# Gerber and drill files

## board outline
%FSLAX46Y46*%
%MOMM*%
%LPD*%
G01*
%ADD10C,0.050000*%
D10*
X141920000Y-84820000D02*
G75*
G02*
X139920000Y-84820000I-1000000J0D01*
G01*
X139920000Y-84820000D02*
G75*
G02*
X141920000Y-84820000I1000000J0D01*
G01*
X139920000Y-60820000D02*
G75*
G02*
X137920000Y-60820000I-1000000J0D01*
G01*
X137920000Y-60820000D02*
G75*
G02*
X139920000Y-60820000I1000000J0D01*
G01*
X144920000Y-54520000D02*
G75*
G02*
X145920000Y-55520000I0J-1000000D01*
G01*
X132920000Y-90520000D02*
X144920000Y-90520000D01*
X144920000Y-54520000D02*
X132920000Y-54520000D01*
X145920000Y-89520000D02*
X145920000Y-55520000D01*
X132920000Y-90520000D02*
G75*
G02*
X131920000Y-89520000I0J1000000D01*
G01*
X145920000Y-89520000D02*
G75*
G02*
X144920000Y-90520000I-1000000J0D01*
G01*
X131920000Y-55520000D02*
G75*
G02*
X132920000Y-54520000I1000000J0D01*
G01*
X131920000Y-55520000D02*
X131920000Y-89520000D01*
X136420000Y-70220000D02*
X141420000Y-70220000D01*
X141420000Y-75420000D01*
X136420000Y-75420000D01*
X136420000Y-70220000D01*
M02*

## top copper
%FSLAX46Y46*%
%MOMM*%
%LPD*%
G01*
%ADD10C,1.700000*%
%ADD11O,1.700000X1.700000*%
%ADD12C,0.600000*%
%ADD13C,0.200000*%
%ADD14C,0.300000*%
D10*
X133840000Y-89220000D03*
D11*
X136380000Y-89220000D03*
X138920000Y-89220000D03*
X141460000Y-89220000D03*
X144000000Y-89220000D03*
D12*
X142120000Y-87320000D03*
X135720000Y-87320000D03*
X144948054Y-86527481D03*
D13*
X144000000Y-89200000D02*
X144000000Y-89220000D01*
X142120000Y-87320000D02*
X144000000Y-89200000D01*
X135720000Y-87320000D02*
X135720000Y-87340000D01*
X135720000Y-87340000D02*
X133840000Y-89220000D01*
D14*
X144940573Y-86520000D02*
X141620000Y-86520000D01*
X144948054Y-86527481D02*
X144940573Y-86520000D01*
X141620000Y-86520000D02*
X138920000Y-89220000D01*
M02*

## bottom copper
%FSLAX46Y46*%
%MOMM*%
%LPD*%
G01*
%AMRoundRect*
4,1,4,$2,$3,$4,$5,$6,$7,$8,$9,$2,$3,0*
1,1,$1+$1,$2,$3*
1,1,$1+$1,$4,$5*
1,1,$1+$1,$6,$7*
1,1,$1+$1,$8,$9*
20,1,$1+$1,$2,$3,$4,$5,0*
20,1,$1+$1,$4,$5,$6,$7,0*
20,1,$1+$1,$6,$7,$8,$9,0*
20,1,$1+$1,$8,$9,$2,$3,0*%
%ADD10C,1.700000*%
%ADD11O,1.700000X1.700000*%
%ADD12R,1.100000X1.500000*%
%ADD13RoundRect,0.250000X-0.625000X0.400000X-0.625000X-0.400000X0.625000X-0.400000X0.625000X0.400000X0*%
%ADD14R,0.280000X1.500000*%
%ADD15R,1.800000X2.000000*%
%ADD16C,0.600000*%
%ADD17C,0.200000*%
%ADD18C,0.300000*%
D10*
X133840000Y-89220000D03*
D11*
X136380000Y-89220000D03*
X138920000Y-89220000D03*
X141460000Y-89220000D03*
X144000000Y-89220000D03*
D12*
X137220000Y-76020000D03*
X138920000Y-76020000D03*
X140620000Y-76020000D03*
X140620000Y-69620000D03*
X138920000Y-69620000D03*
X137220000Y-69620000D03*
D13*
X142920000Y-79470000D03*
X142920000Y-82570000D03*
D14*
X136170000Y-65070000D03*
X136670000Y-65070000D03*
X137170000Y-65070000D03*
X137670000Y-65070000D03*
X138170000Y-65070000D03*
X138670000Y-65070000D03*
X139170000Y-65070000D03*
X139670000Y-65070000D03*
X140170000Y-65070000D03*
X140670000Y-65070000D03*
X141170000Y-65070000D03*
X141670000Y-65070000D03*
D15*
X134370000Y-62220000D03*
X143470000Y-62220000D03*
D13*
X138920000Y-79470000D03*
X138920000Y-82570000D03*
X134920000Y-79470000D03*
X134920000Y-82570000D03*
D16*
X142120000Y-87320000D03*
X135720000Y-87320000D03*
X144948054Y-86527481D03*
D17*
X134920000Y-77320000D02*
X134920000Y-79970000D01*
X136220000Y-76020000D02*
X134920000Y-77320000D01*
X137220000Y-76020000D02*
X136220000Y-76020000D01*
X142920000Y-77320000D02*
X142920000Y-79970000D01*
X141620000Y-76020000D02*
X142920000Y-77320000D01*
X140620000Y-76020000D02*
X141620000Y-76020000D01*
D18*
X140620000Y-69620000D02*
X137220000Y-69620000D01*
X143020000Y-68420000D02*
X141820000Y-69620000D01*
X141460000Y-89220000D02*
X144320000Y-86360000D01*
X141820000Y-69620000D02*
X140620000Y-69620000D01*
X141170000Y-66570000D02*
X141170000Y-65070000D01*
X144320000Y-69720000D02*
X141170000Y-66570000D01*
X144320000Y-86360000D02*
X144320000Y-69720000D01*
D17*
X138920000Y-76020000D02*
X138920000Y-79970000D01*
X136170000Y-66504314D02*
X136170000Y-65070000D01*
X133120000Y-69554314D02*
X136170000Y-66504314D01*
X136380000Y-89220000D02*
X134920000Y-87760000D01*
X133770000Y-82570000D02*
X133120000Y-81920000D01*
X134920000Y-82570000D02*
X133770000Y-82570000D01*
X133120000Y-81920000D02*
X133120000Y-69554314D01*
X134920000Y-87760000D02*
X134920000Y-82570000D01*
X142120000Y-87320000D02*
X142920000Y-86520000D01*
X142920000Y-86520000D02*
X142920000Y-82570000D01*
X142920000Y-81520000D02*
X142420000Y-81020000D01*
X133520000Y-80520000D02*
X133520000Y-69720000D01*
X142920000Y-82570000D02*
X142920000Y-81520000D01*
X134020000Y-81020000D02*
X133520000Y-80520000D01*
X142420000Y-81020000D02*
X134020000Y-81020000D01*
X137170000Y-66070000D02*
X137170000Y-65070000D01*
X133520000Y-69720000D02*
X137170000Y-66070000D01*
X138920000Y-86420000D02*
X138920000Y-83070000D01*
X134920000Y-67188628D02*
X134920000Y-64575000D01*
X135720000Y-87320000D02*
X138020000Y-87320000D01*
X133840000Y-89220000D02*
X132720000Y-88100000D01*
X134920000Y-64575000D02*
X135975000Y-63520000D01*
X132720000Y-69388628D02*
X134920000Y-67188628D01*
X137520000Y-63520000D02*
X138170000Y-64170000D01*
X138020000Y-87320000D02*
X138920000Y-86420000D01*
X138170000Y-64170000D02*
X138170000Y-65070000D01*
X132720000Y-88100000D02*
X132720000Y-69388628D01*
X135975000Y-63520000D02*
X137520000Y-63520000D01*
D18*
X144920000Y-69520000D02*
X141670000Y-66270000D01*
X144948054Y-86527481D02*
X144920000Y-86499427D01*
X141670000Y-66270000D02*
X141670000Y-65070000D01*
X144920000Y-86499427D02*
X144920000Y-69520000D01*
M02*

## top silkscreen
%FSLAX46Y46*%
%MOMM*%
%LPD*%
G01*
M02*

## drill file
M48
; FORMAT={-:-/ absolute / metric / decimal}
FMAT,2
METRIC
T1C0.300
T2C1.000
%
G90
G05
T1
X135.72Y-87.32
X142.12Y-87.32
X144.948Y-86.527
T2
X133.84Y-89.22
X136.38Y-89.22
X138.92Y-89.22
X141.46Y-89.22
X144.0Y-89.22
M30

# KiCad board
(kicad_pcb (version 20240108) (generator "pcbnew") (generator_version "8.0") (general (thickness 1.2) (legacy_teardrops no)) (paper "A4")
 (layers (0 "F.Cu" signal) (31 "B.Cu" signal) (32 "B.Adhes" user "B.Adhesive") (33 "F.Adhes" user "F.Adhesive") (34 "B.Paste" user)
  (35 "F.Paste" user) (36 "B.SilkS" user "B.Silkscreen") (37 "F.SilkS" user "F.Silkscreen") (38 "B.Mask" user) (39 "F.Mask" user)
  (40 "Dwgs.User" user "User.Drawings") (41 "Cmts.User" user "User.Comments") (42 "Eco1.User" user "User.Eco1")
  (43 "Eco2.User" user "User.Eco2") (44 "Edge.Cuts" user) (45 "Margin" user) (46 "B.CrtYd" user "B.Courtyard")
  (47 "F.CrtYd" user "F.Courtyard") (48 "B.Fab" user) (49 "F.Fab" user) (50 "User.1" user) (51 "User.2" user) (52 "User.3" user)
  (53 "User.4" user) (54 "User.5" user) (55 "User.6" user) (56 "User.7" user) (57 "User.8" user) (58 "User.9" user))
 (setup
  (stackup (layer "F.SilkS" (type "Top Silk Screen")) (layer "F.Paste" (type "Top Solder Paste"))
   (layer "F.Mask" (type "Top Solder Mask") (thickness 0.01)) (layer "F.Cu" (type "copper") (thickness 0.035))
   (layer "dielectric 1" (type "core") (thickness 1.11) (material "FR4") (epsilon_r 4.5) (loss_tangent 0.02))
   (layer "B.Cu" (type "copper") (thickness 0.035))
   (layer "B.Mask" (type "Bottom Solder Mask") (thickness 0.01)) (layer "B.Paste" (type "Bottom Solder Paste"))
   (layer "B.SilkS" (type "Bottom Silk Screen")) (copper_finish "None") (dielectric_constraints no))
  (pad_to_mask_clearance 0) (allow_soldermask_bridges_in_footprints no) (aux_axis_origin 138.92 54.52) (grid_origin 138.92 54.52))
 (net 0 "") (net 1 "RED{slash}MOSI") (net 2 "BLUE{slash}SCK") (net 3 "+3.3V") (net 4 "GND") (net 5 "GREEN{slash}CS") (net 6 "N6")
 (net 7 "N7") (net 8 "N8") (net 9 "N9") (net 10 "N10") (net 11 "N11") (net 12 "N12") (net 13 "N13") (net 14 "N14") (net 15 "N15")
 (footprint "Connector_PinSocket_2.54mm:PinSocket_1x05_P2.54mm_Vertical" (layer "F.Cu") (at 133.84 89.22 90)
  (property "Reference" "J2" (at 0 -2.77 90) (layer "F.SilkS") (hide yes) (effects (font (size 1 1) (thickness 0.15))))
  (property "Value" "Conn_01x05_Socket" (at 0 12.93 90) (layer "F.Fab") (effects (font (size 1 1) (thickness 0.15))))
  (pad "1" thru_hole circle (at 0 0 90) (size 1.7 1.7) (drill 1) (layers "*.Cu" "*.Mask") (remove_unused_layers no) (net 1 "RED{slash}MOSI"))
  (pad "2" thru_hole oval (at 0 2.54 90) (size 1.7 1.7) (drill 1) (layers "*.Cu" "*.Mask") (remove_unused_layers no)
   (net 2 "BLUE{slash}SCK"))
  (pad "3" thru_hole oval (at 0 5.08 90) (size 1.7 1.7) (drill 1) (layers "*.Cu" "*.Mask") (remove_unused_layers no) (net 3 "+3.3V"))
  (pad "4" thru_hole oval (at 0 7.62 90) (size 1.7 1.7) (drill 1) (layers "*.Cu" "*.Mask") (remove_unused_layers no) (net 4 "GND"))
  (pad "5" thru_hole oval (at 0 10.16 90) (size 1.7 1.7) (drill 1) (layers "*.Cu" "*.Mask") (remove_unused_layers no)
   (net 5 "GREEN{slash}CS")))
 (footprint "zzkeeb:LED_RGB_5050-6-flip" (layer "F.Cu") (at 138.92 72.82 90)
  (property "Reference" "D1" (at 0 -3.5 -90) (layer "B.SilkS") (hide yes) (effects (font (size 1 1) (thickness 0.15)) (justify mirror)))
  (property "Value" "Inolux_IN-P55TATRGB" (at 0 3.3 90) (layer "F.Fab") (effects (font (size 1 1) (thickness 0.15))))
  (fp_rect (start -2.6 -2.5) (end 2.6 2.5) (stroke (width 0.05) (type default)) (fill none) (layer "Edge.Cuts"))
  (pad "1" smd rect (at -3.2 -1.7) (size 1.1 1.5) (layers "B.Cu" "B.Paste" "B.Mask") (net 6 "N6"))
  (pad "2" smd rect (at -3.2 0) (size 1.1 1.5) (layers "B.Cu" "B.Paste" "B.Mask") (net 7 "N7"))
  (pad "3" smd rect (at -3.2 1.7) (size 1.1 1.5) (layers "B.Cu" "B.Paste" "B.Mask") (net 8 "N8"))
  (pad "4" smd rect (at 3.2 1.7) (size 1.1 1.5) (layers "B.Cu" "B.Paste" "B.Mask") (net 4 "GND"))
  (pad "5" smd rect (at 3.2 0) (size 1.1 1.5) (layers "B.Cu" "B.Paste" "B.Mask") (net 4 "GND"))
  (pad "6" smd rect (at 3.2 -1.7) (size 1.1 1.5) (layers "B.Cu" "B.Paste" "B.Mask") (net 4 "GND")))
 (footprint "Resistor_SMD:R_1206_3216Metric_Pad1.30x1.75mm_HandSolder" (layer "B.Cu") (at 142.92 81.02 -90)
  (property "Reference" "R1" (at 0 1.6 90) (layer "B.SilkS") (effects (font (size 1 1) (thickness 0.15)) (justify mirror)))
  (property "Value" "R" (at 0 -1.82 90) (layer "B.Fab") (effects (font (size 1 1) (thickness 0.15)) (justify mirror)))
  (pad "1" smd roundrect (at -1.55 0 270) (size 1.3 1.75) (layers "B.Cu" "B.Paste" "B.Mask") (roundrect_rratio 0.192308) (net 8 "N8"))
  (pad "2" smd roundrect (at 1.55 0 270) (size 1.3 1.75) (layers "B.Cu" "B.Paste" "B.Mask") (roundrect_rratio 0.192308)
   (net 5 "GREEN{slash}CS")))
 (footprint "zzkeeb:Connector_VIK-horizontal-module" (layer "B.Cu") (at 138.92 63.52)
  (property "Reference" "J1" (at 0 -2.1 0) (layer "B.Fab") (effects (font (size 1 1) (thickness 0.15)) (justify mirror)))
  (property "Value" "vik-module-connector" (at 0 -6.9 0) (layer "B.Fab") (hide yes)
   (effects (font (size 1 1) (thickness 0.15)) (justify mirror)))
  (pad "1" smd rect (at -2.75 1.55) (size 0.28 1.5) (layers "B.Cu" "B.Paste" "B.Mask") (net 2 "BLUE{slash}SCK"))
  (pad "2" smd rect (at -2.25 1.55) (size 0.28 1.5) (layers "B.Cu" "B.Paste" "B.Mask") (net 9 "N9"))
  (pad "3" smd rect (at -1.75 1.55) (size 0.28 1.5) (layers "B.Cu" "B.Paste" "B.Mask") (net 5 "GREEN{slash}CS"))
  (pad "4" smd rect (at -1.25 1.55) (size 0.28 1.5) (layers "B.Cu" "B.Paste" "B.Mask") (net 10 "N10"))
  (pad "5" smd rect (at -0.75 1.55) (size 0.28 1.5) (layers "B.Cu" "B.Paste" "B.Mask") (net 1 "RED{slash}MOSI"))
  (pad "6" smd rect (at -0.25 1.55) (size 0.28 1.5) (layers "B.Cu" "B.Paste" "B.Mask") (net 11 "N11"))
  (pad "7" smd rect (at 0.25 1.55) (size 0.28 1.5) (layers "B.Cu" "B.Paste" "B.Mask") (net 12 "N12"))
  (pad "8" smd rect (at 0.75 1.55) (size 0.28 1.5) (layers "B.Cu" "B.Paste" "B.Mask") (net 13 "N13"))
  (pad "9" smd rect (at 1.25 1.55) (size 0.28 1.5) (layers "B.Cu" "B.Paste" "B.Mask") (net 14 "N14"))
  (pad "10" smd rect (at 1.75 1.55) (size 0.28 1.5) (layers "B.Cu" "B.Paste" "B.Mask") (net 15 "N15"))
  (pad "11" smd rect (at 2.25 1.55) (size 0.28 1.5) (layers "B.Cu" "B.Paste" "B.Mask") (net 4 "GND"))
  (pad "12" smd rect (at 2.75 1.55) (size 0.28 1.5) (layers "B.Cu" "B.Paste" "B.Mask") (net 3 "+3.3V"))
  (pad "MP" smd rect (at -4.55 -1.3) (size 1.8 2) (layers "B.Cu" "B.Paste" "B.Mask"))
  (pad "MP" smd rect (at 4.55 -1.3) (size 1.8 2) (layers "B.Cu" "B.Paste" "B.Mask")))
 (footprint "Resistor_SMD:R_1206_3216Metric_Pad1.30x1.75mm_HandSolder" (layer "B.Cu") (at 138.92 81.02 -90)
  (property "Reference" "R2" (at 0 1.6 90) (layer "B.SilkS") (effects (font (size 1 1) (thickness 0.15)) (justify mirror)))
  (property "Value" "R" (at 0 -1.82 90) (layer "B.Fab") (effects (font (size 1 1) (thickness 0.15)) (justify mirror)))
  (pad "1" smd roundrect (at -1.55 0 270) (size 1.3 1.75) (layers "B.Cu" "B.Paste" "B.Mask") (roundrect_rratio 0.192308) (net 7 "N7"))
  (pad "2" smd roundrect (at 1.55 0 270) (size 1.3 1.75) (layers "B.Cu" "B.Paste" "B.Mask") (roundrect_rratio 0.192308)
   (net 1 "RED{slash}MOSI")))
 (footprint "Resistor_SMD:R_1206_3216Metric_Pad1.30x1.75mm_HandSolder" (layer "B.Cu") (at 134.92 81.02 -90)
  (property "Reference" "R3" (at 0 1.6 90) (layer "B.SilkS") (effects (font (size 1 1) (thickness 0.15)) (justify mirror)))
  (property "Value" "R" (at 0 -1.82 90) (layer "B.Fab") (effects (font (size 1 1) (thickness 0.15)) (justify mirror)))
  (pad "1" smd roundrect (at -1.55 0 270) (size 1.3 1.75) (layers "B.Cu" "B.Paste" "B.Mask") (roundrect_rratio 0.192308) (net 6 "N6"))
  (pad "2" smd roundrect (at 1.55 0 270) (size 1.3 1.75) (layers "B.Cu" "B.Paste" "B.Mask") (roundrect_rratio 0.192308)
   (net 2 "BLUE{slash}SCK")))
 (gr_circle (center 140.92 84.82) (end 141.92 84.82) (stroke (width 0.05) (type default)) (fill none) (layer "Edge.Cuts"))
 (gr_circle (center 138.92 60.82) (end 139.92 60.82) (stroke (width 0.05) (type default)) (fill none) (layer "Edge.Cuts"))
 (gr_arc (start 144.92 54.52) (mid 145.627107 54.812893) (end 145.92 55.52) (stroke (width 0.05) (type default)) (layer "Edge.Cuts"))
 (gr_line (start 132.92 90.52) (end 144.92 90.52) (stroke (width 0.05) (type default)) (layer "Edge.Cuts"))
 (gr_line (start 144.92 54.52) (end 132.92 54.52) (stroke (width 0.05) (type default)) (layer "Edge.Cuts"))
 (gr_line (start 145.92 89.52) (end 145.92 55.52) (stroke (width 0.05) (type default)) (layer "Edge.Cuts"))
 (gr_arc (start 132.92 90.52) (mid 132.212893 90.227107) (end 131.92 89.52) (stroke (width 0.05) (type default)) (layer "Edge.Cuts"))
 (gr_arc (start 145.92 89.52) (mid 145.627107 90.227107) (end 144.92 90.52) (stroke (width 0.05) (type default)) (layer "Edge.Cuts"))
 (gr_arc (start 131.92 55.52) (mid 132.212893 54.812893) (end 132.92 54.52) (stroke (width 0.05) (type default)) (layer "Edge.Cuts"))
 (gr_line (start 131.92 55.52) (end 131.92 89.52) (stroke (width 0.05) (type default)) (layer "Edge.Cuts"))
 (segment (start 134.92 77.32) (end 134.92 79.97) (width 0.2) (layer "B.Cu") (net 6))
 (segment (start 136.22 76.02) (end 134.92 77.32) (width 0.2) (layer "B.Cu") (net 6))
 (segment (start 137.22 76.02) (end 136.22 76.02) (width 0.2) (layer "B.Cu") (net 6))
 (segment (start 142.92 77.32) (end 142.92 79.97) (width 0.2) (layer "B.Cu") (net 8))
 (segment (start 141.62 76.02) (end 142.92 77.32) (width 0.2) (layer "B.Cu") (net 8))
 (segment (start 140.62 76.02) (end 141.62 76.02) (width 0.2) (layer "B.Cu") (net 8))
 (segment (start 140.62 69.62) (end 137.22 69.62) (width 0.3) (layer "B.Cu") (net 4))
 (segment (start 143.02 68.42) (end 141.82 69.62) (width 0.3) (layer "B.Cu") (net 4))
 (segment (start 141.46 89.22) (end 144.32 86.36) (width 0.3) (layer "B.Cu") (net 4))
 (segment (start 141.82 69.62) (end 140.62 69.62) (width 0.3) (layer "B.Cu") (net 4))
 (segment (start 141.17 66.57) (end 141.17 65.07) (width 0.3) (layer "B.Cu") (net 4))
 (segment (start 144.32 69.72) (end 141.17 66.57) (width 0.3) (layer "B.Cu") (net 4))
 (segment (start 144.32 86.36) (end 144.32 69.72) (width 0.3) (layer "B.Cu") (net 4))
 (segment (start 138.92 76.02) (end 138.92 79.97) (width 0.2) (layer "B.Cu") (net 7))
 (segment (start 136.17 66.504314) (end 136.17 65.07) (width 0.2) (layer "B.Cu") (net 2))
 (segment (start 133.12 69.554314) (end 136.17 66.504314) (width 0.2) (layer "B.Cu") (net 2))
 (segment (start 136.38 89.22) (end 134.92 87.76) (width 0.2) (layer "B.Cu") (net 2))
 (segment (start 133.77 82.57) (end 133.12 81.92) (width 0.2) (layer "B.Cu") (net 2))
 (segment (start 134.92 82.57) (end 133.77 82.57) (width 0.2) (layer "B.Cu") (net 2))
 (segment (start 133.12 81.92) (end 133.12 69.554314) (width 0.2) (layer "B.Cu") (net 2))
 (segment (start 134.92 87.76) (end 134.92 82.57) (width 0.2) (layer "B.Cu") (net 2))
 (segment (start 144 89.2) (end 144 89.22) (width 0.2) (layer "F.Cu") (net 5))
 (segment (start 142.12 87.32) (end 144 89.2) (width 0.2) (layer "F.Cu") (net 5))
 (via (at 142.12 87.32) (size 0.6) (drill 0.3) (layers "F.Cu" "B.Cu") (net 5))
 (segment (start 142.12 87.32) (end 142.92 86.52) (width 0.2) (layer "B.Cu") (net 5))
 (segment (start 142.92 86.52) (end 142.92 82.57) (width 0.2) (layer "B.Cu") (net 5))
 (segment (start 142.92 81.52) (end 142.42 81.02) (width 0.2) (layer "B.Cu") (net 5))
 (segment (start 133.52 80.52) (end 133.52 69.72) (width 0.2) (layer "B.Cu") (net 5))
 (segment (start 142.92 82.57) (end 142.92 81.52) (width 0.2) (layer "B.Cu") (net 5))
 (segment (start 134.02 81.02) (end 133.52 80.52) (width 0.2) (layer "B.Cu") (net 5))
 (segment (start 142.42 81.02) (end 134.02 81.02) (width 0.2) (layer "B.Cu") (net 5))
 (segment (start 137.17 66.07) (end 137.17 65.07) (width 0.2) (layer "B.Cu") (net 5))
 (segment (start 133.52 69.72) (end 137.17 66.07) (width 0.2) (layer "B.Cu") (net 5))
 (segment (start 135.72 87.32) (end 135.72 87.34) (width 0.2) (layer "F.Cu") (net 1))
 (segment (start 135.72 87.34) (end 133.84 89.22) (width 0.2) (layer "F.Cu") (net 1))
 (via (at 135.72 87.32) (size 0.6) (drill 0.3) (layers "F.Cu" "B.Cu") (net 1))
 (segment (start 138.92 86.42) (end 138.92 83.07) (width 0.2) (layer "B.Cu") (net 1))
 (segment (start 134.92 67.188628) (end 134.92 64.575) (width 0.2) (layer "B.Cu") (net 1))
 (segment (start 135.72 87.32) (end 138.02 87.32) (width 0.2) (layer "B.Cu") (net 1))
 (segment (start 133.84 89.22) (end 132.72 88.1) (width 0.2) (layer "B.Cu") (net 1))
 (segment (start 134.92 64.575) (end 135.975 63.52) (width 0.2) (layer "B.Cu") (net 1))
 (segment (start 132.72 69.388628) (end 134.92 67.188628) (width 0.2) (layer "B.Cu") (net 1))
 (segment (start 137.52 63.52) (end 138.17 64.17) (width 0.2) (layer "B.Cu") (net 1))
 (segment (start 138.02 87.32) (end 138.92 86.42) (width 0.2) (layer "B.Cu") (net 1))
 (segment (start 138.17 64.17) (end 138.17 65.07) (width 0.2) (layer "B.Cu") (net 1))
 (segment (start 132.72 88.1) (end 132.72 69.388628) (width 0.2) (layer "B.Cu") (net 1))
 (segment (start 135.975 63.52) (end 137.52 63.52) (width 0.2) (layer "B.Cu") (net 1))
 (segment (start 144.940573 86.52) (end 141.62 86.52) (width 0.3) (layer "F.Cu") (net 3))
 (segment (start 144.948054 86.527481) (end 144.940573 86.52) (width 0.3) (layer "F.Cu") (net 3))
 (segment (start 141.62 86.52) (end 138.92 89.22) (width 0.3) (layer "F.Cu") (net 3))
 (via (at 144.948054 86.527481) (size 0.6) (drill 0.3) (layers "F.Cu" "B.Cu") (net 3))
 (segment (start 144.92 69.52) (end 141.67 66.27) (width 0.3) (layer "B.Cu") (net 3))
 (segment (start 144.948054 86.527481) (end 144.92 86.499427) (width 0.3) (layer "B.Cu") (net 3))
 (segment (start 141.67 66.27) (end 141.67 65.07) (width 0.3) (layer "B.Cu") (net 3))
 (segment (start 144.92 86.499427) (end 144.92 69.52) (width 0.3) (layer "B.Cu") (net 3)))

